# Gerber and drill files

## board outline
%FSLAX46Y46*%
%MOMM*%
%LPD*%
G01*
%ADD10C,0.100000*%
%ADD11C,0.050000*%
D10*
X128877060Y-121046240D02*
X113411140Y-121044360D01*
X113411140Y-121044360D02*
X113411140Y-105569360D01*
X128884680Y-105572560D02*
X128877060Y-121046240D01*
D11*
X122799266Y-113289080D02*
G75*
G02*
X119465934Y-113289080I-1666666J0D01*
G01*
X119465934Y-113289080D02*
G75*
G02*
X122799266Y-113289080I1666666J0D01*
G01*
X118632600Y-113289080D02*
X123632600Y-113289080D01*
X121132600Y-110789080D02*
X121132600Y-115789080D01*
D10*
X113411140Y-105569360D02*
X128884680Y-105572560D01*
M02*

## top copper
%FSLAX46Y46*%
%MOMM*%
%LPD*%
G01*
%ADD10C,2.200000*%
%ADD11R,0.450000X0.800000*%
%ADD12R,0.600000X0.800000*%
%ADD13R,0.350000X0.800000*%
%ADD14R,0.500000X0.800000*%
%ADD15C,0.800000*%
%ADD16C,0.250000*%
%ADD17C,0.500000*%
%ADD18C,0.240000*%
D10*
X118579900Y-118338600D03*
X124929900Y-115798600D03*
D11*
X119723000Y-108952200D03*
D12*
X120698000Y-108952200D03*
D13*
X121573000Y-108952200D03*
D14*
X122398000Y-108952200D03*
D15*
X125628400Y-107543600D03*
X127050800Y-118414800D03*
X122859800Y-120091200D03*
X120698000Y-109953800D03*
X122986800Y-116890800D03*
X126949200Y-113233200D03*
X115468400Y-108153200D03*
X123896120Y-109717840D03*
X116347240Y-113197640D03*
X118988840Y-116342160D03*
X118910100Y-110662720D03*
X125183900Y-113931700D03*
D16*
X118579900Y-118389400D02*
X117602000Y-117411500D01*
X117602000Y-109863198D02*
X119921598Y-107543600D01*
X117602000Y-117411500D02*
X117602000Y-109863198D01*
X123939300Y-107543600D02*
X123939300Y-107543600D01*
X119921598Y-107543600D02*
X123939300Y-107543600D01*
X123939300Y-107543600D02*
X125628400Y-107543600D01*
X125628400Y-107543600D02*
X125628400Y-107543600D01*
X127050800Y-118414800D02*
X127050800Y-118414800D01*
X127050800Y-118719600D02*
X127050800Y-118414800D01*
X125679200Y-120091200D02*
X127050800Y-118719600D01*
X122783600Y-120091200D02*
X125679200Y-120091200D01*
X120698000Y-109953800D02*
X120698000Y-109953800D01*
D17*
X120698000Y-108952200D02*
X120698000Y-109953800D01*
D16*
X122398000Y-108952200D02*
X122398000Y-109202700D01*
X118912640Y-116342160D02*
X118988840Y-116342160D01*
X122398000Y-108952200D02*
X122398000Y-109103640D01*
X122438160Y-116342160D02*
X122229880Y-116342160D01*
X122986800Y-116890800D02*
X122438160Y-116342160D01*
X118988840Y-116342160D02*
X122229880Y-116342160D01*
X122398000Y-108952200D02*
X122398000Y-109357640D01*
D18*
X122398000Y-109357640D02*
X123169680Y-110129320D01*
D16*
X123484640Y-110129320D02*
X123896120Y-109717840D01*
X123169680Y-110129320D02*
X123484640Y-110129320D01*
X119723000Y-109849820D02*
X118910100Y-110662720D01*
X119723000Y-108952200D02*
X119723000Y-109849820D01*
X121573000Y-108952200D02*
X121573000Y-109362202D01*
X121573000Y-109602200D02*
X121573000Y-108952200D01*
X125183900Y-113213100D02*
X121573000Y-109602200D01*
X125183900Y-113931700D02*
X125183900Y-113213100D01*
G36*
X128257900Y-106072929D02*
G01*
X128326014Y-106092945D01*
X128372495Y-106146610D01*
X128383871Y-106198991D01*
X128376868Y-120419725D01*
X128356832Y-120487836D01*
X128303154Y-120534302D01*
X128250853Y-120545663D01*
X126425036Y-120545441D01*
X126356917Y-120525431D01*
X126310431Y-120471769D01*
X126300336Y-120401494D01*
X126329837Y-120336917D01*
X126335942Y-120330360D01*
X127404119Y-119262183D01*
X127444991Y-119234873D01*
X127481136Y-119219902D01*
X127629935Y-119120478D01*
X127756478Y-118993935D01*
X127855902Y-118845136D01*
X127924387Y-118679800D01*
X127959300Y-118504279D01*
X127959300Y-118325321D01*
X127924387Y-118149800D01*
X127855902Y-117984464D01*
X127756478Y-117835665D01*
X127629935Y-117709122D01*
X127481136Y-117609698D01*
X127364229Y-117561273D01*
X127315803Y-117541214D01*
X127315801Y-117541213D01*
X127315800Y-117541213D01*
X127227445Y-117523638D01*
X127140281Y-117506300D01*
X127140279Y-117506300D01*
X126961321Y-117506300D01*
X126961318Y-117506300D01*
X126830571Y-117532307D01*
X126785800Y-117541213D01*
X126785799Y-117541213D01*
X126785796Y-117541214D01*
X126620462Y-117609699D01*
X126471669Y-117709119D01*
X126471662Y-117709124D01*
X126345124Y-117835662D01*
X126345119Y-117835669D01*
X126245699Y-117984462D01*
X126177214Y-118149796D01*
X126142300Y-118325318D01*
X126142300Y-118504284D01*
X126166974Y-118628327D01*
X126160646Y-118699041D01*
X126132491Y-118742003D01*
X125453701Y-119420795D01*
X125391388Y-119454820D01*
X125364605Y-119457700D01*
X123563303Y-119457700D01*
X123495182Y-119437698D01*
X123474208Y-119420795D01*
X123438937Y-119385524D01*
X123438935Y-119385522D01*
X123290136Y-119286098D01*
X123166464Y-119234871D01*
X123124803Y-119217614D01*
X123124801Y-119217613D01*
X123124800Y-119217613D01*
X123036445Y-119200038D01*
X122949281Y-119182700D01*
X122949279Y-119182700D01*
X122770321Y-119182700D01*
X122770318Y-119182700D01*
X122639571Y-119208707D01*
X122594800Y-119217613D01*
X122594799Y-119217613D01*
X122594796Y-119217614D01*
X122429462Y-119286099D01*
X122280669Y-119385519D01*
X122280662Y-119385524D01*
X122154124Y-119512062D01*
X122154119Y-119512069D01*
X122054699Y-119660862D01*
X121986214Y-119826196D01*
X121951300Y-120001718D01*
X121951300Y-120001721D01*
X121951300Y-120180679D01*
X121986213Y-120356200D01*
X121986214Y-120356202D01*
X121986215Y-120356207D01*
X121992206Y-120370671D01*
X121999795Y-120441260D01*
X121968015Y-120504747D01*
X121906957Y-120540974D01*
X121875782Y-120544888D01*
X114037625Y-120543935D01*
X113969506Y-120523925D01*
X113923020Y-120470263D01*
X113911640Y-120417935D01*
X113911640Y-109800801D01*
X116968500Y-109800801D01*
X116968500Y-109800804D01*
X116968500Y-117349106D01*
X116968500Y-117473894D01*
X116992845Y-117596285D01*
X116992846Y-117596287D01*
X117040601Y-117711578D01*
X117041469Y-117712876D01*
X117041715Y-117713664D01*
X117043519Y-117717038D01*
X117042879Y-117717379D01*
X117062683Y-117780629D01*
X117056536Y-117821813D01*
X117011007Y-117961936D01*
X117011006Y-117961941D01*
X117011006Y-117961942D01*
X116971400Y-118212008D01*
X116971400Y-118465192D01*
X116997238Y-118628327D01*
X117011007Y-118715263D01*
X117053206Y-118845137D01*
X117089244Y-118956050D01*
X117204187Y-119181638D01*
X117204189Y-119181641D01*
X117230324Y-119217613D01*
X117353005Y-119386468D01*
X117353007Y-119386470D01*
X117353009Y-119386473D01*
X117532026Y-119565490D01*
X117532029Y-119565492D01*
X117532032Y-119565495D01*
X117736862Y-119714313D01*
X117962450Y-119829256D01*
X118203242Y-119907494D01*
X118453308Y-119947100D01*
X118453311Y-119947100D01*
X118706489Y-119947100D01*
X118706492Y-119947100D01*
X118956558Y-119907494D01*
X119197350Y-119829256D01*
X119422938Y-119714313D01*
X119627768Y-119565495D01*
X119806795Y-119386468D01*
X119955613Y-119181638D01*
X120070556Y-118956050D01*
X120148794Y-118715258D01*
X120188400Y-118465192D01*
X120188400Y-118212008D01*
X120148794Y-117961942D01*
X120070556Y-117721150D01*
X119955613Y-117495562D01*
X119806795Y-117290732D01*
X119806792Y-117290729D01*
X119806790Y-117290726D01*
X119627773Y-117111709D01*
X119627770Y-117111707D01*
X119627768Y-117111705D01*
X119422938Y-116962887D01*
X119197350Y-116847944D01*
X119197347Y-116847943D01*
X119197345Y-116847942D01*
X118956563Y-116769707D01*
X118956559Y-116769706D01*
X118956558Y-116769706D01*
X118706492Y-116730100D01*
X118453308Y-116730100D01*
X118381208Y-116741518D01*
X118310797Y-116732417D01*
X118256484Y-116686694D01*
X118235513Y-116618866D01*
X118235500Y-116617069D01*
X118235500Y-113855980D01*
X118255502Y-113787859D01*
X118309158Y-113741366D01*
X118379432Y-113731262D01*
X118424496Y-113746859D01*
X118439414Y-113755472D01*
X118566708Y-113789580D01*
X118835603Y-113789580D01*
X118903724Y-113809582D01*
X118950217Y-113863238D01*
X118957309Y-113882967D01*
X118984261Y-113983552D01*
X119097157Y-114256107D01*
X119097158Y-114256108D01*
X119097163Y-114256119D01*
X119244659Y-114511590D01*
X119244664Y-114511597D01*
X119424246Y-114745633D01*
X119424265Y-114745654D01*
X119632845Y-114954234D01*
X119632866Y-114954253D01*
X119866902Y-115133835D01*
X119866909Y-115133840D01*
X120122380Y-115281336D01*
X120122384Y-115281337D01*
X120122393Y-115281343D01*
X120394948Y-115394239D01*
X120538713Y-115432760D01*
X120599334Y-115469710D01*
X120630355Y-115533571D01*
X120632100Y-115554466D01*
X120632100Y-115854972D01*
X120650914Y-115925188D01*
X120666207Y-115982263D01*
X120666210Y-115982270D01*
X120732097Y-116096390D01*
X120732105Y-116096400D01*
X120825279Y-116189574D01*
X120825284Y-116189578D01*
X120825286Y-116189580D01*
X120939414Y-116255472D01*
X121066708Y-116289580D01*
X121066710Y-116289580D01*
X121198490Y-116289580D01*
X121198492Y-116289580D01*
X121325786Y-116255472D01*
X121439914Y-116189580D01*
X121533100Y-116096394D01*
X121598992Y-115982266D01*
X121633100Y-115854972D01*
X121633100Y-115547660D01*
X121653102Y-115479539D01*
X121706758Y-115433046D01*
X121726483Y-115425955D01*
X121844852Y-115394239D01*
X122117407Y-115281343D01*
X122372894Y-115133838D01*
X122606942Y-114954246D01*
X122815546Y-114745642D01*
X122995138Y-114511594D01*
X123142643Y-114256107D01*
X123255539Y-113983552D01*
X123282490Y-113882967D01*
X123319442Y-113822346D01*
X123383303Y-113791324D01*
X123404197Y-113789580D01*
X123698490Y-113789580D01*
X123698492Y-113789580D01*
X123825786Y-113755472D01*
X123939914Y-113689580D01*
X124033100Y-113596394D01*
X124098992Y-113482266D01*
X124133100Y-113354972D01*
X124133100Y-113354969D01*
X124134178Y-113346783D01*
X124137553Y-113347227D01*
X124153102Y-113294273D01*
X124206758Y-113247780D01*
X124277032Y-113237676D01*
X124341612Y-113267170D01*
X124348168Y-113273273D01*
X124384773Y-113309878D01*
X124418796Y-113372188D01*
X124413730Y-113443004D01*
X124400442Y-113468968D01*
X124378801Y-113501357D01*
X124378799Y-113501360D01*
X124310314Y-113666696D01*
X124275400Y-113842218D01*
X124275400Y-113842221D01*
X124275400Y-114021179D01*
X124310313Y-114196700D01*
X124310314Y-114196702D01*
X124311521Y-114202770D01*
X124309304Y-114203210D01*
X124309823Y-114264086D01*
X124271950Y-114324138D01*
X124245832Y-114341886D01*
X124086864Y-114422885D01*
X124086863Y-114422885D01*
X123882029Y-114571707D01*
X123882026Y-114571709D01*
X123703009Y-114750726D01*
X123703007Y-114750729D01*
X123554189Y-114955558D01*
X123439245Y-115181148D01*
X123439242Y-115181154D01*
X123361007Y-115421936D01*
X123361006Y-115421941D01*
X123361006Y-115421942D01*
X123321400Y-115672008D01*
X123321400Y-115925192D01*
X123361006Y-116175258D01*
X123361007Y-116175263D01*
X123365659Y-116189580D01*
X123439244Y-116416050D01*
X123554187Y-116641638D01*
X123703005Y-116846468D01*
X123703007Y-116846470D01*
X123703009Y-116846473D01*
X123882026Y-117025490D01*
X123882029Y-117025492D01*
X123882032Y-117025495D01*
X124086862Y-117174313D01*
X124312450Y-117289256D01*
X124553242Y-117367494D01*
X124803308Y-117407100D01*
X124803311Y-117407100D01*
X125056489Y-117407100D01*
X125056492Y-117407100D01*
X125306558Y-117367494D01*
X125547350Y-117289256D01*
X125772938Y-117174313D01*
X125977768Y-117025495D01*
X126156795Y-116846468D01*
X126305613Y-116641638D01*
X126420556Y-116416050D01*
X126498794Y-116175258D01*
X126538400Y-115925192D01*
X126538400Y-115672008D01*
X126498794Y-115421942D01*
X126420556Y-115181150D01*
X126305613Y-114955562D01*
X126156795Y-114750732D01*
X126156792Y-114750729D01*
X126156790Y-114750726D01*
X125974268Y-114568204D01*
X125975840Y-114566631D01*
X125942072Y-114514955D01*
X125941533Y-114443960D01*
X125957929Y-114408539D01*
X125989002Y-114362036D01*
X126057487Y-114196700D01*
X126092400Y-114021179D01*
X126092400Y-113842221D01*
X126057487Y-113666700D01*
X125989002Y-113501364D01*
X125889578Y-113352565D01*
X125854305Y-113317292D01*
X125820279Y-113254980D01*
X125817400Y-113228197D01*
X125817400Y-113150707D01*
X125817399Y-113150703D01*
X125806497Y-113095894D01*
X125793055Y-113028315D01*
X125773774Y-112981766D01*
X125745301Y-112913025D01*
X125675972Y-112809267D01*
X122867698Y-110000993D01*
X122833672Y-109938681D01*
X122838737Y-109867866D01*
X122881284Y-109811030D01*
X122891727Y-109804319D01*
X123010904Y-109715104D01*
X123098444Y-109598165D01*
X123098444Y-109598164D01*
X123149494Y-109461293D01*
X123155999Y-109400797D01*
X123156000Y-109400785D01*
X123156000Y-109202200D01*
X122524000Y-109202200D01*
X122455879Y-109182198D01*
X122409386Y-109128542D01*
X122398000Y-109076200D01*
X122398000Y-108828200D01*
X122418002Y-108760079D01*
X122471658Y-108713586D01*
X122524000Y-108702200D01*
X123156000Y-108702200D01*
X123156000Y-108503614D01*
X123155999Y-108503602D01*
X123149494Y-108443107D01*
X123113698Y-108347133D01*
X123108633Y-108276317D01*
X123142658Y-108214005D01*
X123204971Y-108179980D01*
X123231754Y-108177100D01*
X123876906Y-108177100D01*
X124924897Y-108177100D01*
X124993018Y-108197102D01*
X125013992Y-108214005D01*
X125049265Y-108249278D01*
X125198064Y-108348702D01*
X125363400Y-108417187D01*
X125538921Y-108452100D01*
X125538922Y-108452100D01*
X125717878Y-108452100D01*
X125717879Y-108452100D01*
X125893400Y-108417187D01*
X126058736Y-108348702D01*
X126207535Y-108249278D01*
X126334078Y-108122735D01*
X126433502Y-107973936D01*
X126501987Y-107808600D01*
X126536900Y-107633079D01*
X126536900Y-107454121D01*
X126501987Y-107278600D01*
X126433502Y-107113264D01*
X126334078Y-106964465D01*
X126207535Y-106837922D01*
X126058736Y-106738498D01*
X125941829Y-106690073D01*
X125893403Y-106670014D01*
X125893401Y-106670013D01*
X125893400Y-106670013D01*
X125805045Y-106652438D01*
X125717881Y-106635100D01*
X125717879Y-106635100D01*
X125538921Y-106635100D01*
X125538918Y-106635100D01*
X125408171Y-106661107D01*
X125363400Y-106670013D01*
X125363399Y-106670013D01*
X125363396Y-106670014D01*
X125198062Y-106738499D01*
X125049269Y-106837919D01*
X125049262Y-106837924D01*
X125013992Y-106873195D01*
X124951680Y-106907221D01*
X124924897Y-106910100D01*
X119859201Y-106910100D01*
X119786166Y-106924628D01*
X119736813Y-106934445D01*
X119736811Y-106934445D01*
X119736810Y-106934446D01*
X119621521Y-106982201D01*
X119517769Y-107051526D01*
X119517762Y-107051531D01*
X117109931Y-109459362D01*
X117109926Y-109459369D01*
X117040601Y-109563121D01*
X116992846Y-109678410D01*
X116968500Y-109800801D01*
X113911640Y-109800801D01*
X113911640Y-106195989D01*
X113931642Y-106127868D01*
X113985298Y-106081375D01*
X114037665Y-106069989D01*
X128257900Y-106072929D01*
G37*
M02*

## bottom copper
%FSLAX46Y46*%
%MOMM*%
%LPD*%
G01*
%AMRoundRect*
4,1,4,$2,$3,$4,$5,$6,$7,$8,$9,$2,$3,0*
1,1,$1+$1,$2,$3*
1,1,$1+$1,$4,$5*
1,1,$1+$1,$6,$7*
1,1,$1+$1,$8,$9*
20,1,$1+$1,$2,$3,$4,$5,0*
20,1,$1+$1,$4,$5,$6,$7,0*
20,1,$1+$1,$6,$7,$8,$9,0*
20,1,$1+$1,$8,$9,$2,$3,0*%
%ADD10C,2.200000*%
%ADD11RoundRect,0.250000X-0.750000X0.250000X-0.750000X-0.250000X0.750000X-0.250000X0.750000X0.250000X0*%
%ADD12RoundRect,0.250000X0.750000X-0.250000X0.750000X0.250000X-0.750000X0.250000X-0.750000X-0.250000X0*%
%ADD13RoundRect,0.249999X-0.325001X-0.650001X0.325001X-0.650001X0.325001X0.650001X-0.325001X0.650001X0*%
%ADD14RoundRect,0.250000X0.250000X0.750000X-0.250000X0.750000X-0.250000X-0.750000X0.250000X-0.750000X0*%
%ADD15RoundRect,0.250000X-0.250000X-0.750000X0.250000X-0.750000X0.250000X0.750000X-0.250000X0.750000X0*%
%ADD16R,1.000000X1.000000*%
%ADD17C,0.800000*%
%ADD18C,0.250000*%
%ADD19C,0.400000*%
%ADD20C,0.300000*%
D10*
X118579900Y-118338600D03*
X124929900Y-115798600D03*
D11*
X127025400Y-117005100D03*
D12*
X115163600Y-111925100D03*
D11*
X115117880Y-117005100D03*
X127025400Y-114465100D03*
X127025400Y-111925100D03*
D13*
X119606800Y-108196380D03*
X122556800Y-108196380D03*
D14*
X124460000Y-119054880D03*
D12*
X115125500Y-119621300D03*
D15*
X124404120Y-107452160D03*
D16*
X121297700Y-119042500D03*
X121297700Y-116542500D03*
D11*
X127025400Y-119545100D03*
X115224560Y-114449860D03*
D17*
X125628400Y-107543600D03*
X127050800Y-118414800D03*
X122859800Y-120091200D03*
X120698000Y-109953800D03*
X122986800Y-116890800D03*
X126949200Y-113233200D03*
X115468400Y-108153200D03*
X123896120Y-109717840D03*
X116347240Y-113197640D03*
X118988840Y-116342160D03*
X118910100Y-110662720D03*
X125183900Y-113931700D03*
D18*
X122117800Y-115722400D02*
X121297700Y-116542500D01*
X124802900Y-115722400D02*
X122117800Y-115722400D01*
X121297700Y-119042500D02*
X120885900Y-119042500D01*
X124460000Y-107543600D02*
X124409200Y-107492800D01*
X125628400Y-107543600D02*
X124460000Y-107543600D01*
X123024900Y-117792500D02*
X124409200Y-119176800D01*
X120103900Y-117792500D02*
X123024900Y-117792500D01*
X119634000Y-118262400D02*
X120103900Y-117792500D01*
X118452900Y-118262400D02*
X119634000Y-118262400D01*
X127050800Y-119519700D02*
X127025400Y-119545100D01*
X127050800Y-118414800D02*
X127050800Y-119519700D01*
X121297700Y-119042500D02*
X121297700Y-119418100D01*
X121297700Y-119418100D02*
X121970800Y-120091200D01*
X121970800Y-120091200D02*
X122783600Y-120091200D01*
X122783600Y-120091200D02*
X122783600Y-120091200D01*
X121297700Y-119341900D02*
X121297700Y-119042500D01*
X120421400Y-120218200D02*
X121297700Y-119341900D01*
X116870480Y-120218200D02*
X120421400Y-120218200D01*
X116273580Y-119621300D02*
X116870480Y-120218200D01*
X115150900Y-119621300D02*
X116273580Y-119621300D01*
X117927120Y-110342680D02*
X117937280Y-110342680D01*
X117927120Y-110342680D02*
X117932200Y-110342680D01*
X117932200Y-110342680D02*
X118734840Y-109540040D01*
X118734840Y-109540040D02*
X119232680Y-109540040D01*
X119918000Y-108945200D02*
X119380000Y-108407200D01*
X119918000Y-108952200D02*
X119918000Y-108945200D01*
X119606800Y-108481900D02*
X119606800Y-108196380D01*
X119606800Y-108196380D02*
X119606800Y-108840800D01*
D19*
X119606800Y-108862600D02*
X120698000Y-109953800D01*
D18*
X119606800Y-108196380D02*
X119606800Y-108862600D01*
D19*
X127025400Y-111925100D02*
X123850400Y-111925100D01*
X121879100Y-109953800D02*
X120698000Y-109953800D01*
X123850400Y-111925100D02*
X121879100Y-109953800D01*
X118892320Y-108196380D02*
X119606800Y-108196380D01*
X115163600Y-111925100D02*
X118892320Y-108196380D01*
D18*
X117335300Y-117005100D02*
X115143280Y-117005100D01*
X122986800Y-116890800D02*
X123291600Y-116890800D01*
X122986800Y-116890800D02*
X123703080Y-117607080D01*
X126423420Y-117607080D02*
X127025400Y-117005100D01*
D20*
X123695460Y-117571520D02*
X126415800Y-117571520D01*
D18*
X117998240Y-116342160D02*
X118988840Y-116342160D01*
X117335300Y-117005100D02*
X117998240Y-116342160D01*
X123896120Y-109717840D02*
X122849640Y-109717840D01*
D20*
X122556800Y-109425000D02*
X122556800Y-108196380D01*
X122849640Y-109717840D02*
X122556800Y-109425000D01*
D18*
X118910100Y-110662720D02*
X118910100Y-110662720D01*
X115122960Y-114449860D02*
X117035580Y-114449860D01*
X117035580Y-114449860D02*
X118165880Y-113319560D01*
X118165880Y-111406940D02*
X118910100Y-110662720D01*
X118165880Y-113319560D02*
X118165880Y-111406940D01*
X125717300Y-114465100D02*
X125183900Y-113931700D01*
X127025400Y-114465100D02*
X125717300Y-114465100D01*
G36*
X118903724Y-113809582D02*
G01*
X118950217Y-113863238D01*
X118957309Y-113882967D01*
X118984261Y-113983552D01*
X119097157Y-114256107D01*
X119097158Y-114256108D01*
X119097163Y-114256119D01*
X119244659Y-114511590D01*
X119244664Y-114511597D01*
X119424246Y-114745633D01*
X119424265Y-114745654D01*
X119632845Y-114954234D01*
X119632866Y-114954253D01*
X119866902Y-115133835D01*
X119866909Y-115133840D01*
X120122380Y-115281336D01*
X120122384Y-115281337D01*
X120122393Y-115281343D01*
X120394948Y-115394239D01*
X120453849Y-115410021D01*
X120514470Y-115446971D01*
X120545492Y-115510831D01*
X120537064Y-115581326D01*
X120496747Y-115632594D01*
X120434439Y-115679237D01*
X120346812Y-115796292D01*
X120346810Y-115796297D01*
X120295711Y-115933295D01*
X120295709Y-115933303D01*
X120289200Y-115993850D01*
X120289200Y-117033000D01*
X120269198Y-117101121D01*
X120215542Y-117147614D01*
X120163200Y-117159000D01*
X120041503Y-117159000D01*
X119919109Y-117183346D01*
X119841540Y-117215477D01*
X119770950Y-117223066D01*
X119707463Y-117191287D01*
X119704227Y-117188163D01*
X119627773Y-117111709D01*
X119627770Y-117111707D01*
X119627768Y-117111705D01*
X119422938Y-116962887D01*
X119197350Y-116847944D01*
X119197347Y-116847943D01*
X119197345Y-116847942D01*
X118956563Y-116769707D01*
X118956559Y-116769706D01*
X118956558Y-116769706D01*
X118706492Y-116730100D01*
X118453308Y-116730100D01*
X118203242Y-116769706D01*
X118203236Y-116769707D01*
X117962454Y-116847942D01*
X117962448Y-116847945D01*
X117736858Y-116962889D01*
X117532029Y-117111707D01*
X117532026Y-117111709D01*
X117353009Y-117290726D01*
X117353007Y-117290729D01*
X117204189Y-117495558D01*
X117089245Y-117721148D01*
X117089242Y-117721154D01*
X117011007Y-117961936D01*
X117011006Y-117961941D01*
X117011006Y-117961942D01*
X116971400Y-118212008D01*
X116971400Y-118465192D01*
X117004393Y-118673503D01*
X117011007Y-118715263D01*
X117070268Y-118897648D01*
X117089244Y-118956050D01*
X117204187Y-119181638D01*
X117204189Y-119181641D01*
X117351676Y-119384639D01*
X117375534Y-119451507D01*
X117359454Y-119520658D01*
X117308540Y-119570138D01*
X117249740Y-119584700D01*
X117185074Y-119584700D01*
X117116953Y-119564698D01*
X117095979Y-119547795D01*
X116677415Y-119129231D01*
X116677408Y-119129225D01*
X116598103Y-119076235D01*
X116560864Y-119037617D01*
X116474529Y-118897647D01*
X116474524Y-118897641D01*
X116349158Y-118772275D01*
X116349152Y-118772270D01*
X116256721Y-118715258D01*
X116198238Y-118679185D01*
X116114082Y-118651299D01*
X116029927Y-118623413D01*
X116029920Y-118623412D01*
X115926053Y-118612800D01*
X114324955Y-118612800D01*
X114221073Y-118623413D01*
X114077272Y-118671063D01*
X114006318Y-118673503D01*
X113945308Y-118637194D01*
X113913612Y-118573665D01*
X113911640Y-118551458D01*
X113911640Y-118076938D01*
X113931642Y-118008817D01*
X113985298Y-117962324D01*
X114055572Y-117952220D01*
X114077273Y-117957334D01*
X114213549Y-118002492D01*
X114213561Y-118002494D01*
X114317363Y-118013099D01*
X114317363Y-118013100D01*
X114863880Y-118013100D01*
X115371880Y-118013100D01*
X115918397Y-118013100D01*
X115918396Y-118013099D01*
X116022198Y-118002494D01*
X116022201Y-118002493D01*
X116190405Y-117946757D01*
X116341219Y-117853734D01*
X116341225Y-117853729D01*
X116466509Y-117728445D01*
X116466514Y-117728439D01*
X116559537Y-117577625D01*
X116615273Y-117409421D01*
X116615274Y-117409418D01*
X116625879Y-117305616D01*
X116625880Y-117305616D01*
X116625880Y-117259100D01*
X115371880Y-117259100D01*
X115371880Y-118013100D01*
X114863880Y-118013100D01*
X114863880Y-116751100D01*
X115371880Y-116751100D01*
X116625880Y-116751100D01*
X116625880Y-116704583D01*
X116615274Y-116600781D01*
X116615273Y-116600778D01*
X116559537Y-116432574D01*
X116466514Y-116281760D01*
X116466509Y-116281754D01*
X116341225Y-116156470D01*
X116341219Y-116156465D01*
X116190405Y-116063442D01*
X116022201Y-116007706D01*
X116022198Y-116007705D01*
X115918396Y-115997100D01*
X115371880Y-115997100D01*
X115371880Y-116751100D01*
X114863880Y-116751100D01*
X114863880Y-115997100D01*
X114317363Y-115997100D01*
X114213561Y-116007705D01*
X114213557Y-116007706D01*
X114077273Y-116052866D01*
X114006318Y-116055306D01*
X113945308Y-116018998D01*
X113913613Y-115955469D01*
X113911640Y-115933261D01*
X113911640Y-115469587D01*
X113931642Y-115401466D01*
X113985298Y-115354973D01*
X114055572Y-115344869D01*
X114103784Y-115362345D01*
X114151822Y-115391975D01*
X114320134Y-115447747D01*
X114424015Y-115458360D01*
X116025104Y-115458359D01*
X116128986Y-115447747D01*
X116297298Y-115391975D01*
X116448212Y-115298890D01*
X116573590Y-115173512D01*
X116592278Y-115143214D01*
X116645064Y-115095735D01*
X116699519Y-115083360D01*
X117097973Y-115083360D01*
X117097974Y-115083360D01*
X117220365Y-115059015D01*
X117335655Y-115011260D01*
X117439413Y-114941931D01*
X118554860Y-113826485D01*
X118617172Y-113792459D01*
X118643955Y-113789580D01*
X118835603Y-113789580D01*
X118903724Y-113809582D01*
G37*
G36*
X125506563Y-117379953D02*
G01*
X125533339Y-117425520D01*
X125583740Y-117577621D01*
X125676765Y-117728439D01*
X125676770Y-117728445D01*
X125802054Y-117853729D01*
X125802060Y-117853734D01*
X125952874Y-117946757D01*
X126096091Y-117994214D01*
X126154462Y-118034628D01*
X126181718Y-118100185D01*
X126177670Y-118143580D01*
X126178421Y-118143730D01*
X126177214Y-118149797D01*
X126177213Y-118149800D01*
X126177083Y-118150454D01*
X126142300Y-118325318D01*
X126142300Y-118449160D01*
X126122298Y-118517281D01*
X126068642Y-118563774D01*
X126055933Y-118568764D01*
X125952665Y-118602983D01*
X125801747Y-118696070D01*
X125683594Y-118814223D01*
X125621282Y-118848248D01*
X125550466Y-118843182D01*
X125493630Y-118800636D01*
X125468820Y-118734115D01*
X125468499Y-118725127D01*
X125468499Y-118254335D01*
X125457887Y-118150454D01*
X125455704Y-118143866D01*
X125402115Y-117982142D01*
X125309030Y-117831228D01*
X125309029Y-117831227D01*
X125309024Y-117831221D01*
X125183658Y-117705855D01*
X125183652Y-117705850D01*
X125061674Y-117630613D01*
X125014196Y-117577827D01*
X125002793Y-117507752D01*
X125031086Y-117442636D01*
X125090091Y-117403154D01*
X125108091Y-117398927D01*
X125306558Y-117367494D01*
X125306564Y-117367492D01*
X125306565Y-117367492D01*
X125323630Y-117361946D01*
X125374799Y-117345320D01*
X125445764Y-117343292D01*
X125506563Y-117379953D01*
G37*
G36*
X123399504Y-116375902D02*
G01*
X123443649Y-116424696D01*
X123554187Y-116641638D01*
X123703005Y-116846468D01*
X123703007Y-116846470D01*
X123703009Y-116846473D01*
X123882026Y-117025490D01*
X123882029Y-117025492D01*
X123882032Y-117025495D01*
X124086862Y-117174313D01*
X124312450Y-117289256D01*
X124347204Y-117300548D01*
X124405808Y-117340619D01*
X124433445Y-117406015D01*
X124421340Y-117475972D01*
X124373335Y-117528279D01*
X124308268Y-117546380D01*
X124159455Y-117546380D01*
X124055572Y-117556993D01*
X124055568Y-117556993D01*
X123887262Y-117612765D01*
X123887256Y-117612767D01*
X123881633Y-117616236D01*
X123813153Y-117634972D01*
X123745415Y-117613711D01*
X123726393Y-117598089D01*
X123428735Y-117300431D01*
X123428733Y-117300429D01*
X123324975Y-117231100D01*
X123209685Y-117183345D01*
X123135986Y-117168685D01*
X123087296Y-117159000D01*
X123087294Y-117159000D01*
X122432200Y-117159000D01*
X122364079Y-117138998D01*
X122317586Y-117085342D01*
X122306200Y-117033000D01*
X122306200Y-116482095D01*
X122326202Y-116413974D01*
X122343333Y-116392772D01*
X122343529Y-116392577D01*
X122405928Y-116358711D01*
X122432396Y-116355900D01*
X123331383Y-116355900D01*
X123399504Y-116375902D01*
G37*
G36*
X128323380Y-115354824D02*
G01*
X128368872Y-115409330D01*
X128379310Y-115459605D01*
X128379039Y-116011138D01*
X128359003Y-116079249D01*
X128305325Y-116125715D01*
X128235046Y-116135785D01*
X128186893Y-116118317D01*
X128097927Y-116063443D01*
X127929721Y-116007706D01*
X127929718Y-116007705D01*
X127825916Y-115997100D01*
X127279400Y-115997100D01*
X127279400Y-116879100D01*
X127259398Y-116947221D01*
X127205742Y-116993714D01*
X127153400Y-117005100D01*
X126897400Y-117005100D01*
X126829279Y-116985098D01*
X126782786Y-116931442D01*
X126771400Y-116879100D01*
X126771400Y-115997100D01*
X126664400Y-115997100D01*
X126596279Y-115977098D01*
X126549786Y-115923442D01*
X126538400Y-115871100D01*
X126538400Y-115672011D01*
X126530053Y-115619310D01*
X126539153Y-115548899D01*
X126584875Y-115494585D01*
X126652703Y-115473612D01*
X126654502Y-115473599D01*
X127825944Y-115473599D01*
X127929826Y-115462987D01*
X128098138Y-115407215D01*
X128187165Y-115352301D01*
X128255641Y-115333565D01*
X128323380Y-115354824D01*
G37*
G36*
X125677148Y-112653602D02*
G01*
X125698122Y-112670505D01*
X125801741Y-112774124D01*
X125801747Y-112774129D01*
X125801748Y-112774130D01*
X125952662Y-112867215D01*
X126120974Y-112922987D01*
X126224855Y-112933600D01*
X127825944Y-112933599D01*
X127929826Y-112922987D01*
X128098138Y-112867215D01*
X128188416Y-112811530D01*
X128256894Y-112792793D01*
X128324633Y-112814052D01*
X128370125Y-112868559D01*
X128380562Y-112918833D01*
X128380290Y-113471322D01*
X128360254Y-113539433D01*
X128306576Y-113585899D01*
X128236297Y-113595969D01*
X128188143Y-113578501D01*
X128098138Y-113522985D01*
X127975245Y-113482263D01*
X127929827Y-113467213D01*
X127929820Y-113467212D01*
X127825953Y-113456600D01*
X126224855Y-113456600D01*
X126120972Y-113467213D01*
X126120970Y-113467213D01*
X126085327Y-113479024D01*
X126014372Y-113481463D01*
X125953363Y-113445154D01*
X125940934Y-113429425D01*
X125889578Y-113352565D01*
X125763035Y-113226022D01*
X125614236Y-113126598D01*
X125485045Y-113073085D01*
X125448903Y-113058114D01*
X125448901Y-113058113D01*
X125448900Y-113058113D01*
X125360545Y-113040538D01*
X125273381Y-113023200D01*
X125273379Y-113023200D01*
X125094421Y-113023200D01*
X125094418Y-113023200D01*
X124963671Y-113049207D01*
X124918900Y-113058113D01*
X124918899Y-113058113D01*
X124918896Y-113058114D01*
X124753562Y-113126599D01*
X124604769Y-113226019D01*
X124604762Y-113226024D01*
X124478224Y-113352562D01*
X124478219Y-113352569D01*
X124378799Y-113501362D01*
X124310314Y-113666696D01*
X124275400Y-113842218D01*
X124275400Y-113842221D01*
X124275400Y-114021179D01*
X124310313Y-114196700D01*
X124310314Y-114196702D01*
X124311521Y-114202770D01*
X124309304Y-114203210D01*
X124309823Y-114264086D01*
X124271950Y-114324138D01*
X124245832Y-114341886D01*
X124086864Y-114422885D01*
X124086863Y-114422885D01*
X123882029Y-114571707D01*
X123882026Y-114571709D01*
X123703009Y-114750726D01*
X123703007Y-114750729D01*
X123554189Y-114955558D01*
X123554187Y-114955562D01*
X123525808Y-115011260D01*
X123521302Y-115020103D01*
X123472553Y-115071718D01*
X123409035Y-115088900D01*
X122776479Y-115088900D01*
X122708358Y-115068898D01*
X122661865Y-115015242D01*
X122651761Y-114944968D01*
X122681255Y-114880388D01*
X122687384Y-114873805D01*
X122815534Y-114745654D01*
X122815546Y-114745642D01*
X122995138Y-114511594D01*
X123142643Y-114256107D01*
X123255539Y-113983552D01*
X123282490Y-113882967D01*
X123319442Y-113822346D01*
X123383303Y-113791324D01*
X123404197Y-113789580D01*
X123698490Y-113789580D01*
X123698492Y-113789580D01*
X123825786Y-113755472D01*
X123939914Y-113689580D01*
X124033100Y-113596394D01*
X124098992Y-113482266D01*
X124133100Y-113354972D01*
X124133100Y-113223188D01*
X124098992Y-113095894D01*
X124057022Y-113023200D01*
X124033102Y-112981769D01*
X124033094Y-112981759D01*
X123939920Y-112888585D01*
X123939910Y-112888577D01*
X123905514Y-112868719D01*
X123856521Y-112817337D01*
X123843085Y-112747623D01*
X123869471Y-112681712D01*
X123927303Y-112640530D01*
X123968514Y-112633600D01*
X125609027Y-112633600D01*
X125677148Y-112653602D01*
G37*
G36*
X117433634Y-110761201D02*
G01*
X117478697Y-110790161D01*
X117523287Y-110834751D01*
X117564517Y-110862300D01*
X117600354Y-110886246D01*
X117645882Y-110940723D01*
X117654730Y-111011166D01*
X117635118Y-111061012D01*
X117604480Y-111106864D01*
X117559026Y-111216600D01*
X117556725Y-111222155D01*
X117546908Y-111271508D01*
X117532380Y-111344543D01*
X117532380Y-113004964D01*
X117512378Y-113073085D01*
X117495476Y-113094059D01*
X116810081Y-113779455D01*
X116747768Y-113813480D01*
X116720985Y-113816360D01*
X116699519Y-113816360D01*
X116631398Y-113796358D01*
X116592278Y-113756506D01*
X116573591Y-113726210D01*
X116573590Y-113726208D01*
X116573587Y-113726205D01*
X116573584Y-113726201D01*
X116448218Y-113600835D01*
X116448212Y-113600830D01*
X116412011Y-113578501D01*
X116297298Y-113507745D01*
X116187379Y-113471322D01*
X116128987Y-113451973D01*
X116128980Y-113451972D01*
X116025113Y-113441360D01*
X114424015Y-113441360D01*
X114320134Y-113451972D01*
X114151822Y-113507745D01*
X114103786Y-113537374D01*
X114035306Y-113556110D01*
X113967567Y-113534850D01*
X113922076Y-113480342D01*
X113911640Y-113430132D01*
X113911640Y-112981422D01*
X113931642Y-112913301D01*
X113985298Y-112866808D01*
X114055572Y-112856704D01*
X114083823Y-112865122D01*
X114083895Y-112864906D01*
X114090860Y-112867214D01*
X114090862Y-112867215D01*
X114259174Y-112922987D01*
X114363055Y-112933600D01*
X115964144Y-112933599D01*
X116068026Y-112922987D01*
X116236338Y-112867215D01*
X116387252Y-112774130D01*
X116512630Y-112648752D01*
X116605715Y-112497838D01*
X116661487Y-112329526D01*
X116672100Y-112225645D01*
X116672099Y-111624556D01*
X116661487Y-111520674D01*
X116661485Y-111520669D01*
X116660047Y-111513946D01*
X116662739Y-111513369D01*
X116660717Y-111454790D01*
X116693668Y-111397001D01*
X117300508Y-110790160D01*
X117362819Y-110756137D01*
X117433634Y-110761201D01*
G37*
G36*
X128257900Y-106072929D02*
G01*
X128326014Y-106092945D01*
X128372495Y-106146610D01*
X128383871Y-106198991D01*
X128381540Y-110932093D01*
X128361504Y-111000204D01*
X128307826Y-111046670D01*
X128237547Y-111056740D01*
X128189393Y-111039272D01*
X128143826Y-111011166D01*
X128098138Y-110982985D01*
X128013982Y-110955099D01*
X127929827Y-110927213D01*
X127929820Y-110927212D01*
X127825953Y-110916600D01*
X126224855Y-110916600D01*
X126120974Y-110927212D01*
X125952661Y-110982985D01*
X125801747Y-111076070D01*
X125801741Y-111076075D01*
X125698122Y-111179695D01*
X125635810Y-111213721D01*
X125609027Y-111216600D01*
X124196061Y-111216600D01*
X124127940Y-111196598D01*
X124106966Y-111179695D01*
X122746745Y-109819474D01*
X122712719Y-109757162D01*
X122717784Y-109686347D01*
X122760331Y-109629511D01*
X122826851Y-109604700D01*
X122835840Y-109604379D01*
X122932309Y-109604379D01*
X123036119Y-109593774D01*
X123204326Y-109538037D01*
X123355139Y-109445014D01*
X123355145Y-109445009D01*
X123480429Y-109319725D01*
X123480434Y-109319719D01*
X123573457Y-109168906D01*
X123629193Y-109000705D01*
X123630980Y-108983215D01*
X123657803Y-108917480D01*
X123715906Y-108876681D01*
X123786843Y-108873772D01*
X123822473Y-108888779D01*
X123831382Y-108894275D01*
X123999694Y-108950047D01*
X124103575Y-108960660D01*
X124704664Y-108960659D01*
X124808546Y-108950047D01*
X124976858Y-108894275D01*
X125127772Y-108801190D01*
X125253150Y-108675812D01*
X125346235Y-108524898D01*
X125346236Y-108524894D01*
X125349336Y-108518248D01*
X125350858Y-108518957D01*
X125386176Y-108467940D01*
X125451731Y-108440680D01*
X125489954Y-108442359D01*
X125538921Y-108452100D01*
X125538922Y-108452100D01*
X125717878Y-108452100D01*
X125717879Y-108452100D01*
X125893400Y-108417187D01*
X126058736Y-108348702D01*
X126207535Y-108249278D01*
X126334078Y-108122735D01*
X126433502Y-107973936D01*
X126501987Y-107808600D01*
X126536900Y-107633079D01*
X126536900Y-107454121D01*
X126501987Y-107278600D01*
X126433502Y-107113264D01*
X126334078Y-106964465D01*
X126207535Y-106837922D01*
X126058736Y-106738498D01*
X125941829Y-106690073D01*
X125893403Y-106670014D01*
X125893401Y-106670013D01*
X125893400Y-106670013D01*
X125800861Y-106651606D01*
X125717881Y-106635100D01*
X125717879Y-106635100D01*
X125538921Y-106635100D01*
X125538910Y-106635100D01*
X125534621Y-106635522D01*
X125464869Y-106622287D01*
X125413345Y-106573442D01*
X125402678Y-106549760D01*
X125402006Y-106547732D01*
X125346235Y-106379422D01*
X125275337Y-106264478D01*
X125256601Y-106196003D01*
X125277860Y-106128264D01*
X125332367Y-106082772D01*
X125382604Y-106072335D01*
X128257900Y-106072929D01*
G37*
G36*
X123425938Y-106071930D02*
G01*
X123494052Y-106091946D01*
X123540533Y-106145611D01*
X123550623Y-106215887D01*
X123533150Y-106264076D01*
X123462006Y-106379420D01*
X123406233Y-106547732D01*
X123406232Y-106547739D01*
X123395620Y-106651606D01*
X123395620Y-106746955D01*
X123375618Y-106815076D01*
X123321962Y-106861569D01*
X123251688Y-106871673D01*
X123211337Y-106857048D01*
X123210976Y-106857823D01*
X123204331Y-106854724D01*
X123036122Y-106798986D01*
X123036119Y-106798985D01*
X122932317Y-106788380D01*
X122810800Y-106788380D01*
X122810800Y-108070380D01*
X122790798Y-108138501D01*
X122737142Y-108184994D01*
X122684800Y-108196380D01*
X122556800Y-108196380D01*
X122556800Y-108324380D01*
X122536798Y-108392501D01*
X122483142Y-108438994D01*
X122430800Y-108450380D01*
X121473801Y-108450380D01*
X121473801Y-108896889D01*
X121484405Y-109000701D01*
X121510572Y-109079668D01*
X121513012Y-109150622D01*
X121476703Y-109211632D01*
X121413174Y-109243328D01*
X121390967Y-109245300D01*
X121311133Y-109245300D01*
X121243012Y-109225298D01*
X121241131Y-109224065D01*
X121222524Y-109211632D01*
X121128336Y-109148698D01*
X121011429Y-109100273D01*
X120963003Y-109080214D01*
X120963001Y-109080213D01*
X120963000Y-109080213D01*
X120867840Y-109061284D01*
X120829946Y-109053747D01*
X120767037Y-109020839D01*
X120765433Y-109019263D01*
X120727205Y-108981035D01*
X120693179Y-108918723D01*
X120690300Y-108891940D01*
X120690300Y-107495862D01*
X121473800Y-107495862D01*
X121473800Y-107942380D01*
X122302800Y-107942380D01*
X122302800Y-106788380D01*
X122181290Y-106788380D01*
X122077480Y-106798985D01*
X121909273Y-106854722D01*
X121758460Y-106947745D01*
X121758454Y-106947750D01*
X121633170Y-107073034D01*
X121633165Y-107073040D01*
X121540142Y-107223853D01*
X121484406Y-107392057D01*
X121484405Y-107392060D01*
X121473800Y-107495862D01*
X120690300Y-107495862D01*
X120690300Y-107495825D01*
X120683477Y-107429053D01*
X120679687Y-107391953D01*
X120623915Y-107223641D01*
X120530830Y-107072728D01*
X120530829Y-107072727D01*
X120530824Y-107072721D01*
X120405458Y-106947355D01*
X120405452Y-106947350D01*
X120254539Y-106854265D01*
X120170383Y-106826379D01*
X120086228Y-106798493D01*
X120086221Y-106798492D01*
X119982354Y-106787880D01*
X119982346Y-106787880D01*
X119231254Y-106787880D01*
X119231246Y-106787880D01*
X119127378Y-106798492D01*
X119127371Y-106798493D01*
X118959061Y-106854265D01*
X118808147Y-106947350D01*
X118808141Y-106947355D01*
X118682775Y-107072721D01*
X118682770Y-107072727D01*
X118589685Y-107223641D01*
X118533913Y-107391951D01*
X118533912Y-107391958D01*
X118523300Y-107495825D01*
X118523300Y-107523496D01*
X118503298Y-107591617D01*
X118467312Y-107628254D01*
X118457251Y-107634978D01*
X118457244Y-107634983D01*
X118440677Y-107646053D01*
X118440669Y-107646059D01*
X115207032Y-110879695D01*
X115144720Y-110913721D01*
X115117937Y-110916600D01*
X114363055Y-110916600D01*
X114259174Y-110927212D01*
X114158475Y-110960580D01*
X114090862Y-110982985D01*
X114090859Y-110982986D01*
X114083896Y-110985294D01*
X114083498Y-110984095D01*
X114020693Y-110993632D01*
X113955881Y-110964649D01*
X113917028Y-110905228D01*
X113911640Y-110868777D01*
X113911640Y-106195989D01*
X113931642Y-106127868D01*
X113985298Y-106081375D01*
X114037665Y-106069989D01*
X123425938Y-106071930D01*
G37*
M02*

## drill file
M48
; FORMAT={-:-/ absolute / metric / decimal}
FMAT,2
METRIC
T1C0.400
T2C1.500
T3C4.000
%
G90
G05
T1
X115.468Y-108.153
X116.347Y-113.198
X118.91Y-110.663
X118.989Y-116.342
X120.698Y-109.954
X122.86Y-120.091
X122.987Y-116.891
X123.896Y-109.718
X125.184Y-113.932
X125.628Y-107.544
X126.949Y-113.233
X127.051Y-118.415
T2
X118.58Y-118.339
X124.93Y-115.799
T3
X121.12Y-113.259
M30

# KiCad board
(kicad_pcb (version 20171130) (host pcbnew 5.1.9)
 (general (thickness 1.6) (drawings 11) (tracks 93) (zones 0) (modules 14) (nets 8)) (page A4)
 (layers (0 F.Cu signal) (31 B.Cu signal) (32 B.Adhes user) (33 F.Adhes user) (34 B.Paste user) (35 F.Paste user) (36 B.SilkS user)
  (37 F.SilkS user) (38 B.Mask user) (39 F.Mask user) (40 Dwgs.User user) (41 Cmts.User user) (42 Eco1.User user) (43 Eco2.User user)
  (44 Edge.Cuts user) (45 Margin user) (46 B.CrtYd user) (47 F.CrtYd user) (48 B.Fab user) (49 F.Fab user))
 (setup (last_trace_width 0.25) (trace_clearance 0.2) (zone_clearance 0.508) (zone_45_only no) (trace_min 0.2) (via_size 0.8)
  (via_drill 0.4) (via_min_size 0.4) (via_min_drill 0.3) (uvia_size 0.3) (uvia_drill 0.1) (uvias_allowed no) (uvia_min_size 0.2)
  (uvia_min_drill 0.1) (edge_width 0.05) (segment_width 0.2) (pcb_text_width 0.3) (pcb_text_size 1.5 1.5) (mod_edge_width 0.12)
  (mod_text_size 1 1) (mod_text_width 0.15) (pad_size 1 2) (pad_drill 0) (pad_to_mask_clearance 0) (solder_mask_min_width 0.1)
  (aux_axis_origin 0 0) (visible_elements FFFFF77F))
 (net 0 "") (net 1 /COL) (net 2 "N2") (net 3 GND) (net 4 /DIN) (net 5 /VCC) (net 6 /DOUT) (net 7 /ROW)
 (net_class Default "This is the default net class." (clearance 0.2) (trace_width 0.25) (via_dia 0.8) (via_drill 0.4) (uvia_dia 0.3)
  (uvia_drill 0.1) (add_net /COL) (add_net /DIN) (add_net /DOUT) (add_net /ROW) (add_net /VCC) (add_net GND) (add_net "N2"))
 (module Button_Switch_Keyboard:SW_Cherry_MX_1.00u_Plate (layer F.Cu) (at 118.5799 118.3386 180)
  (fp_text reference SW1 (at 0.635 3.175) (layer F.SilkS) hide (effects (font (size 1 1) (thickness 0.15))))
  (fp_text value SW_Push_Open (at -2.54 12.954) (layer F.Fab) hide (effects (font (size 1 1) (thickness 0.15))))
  (pad 1 thru_hole circle (at 0 0 180) (size 2.2 2.2) (drill 1.5) (layers *.Cu *.Mask) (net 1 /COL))
  (pad 2 thru_hole circle (at -6.35 2.54 180) (size 2.2 2.2) (drill 1.5) (layers *.Cu *.Mask) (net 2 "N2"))
  (pad "" np_thru_hole circle (at -2.54 5.08 180) (size 4 4) (drill 4) (layers *.Cu *.Mask)))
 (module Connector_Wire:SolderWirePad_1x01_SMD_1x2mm (layer B.Cu) (at 127.0254 117.0051 270)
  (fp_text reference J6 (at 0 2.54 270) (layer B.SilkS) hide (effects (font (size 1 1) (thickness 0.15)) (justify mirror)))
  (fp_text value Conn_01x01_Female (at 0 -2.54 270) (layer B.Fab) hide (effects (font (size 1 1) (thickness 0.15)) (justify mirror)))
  (pad 1 smd roundrect (at 0 0 270) (size 1 2) (layers B.Cu B.Paste B.Mask) (roundrect_rratio 0.25) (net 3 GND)))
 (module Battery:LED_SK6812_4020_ (layer F.Cu) (at 121.158 107.7722)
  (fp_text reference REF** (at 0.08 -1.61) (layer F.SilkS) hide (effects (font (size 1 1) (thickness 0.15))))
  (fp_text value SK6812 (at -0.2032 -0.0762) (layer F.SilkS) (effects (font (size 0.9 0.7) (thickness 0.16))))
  (pad 1 smd rect (at -1.435 1.18) (size 0.45 0.8) (layers F.Cu F.Paste F.Mask) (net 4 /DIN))
  (pad 2 smd rect (at -0.46 1.18) (size 0.6 0.8) (layers F.Cu F.Paste F.Mask) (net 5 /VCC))
  (pad 3 smd rect (at 0.415 1.18) (size 0.35 0.8) (layers F.Cu F.Paste F.Mask) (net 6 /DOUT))
  (pad 4 smd rect (at 1.24 1.18) (size 0.5 0.8) (layers F.Cu F.Paste F.Mask) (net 3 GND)))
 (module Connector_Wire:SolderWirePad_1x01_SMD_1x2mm (layer B.Cu) (at 115.1636 111.9251 90)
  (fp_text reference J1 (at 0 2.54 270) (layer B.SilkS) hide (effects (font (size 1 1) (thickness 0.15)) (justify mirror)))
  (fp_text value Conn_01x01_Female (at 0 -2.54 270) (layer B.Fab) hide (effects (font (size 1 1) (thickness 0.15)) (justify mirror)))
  (pad 1 smd roundrect (at 0 0 90) (size 1 2) (layers B.Cu B.Paste B.Mask) (roundrect_rratio 0.25) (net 5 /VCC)))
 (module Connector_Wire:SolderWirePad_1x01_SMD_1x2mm (layer B.Cu) (at 115.11788 117.0051 270)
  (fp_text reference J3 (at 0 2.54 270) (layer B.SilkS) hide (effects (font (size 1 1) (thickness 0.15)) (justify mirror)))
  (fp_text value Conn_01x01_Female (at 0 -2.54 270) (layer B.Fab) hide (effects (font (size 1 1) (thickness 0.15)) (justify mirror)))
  (pad 1 smd roundrect (at 0 0 270) (size 1 2) (layers B.Cu B.Paste B.Mask) (roundrect_rratio 0.25) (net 3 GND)))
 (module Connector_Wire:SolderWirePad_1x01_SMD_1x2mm (layer B.Cu) (at 127.0254 114.4651 270)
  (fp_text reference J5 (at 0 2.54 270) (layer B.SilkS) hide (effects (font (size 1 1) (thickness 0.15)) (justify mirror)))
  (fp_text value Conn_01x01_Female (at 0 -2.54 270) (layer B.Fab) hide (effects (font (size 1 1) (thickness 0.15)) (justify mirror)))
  (pad 1 smd roundrect (at 0 0 270) (size 1 2) (layers B.Cu B.Paste B.Mask) (roundrect_rratio 0.25) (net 6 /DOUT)))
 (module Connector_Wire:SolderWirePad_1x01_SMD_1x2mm (layer B.Cu) (at 127.0254 111.9251 270)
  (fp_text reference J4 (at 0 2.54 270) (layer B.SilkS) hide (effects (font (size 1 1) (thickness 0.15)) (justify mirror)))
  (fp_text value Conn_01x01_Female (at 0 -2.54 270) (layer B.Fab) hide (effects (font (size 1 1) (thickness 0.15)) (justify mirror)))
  (pad 1 smd roundrect (at 0 0 270) (size 1 2) (layers B.Cu B.Paste B.Mask) (roundrect_rratio 0.25) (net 5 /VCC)))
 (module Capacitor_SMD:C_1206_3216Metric (layer B.Cu) (at 121.0818 108.19638)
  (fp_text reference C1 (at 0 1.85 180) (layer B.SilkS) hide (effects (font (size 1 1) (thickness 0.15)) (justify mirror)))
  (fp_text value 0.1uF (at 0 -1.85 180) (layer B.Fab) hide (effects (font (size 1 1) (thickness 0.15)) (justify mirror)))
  (pad 1 smd roundrect (at -1.475 0) (size 1.15 1.8) (layers B.Cu B.Paste B.Mask) (roundrect_rratio 0.2173904347826087) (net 5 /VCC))
  (pad 2 smd roundrect (at 1.475 0) (size 1.15 1.8) (layers B.Cu B.Paste B.Mask) (roundrect_rratio 0.2173904347826087) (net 3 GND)))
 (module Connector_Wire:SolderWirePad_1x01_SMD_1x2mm (layer B.Cu) (at 124.46 119.05488 180)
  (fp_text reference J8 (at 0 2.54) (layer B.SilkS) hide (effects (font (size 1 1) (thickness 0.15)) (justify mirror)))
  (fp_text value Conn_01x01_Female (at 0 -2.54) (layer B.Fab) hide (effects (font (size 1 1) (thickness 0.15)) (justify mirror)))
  (pad 1 smd roundrect (at 0 0 180) (size 1 2) (layers B.Cu B.Paste B.Mask) (roundrect_rratio 0.25) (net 1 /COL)))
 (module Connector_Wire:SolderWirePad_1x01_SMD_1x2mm (layer B.Cu) (at 115.1255 119.6213 90)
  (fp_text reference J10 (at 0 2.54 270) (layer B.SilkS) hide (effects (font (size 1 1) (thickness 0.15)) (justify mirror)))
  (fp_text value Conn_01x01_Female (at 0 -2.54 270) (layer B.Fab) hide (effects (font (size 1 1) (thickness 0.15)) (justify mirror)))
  (pad 1 smd roundrect (at 0 0 90) (size 1 2) (layers B.Cu B.Paste B.Mask) (roundrect_rratio 0.25) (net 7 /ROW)))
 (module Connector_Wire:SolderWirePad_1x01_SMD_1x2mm (layer B.Cu) (at 124.40412 107.45216)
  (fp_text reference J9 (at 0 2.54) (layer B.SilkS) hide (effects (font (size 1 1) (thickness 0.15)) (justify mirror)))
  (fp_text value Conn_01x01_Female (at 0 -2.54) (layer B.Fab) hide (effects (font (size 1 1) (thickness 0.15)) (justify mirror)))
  (pad 1 smd roundrect (at 0 0) (size 1 2) (layers B.Cu B.Paste B.Mask) (roundrect_rratio 0.25) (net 1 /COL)))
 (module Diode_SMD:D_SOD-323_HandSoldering (layer B.Cu) (at 121.2977 117.7925 90)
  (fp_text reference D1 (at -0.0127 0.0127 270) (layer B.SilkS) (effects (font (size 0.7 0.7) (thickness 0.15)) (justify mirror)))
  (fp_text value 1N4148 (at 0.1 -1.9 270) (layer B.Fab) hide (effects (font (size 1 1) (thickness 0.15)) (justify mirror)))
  (pad 1 smd rect (at -1.25 0 90) (size 1 1) (layers B.Cu B.Paste B.Mask) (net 7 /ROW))
  (pad 2 smd rect (at 1.25 0 90) (size 1 1) (layers B.Cu B.Paste B.Mask) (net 2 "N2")))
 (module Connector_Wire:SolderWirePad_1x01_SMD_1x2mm (layer B.Cu) (at 127.0254 119.5451 270)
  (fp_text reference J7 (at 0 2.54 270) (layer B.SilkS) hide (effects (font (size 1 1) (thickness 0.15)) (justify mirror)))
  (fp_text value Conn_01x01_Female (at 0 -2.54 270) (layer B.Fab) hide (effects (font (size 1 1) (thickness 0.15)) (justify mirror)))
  (pad 1 smd roundrect (at 0 0 270) (size 1 2) (layers B.Cu B.Paste B.Mask) (roundrect_rratio 0.25) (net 7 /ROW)))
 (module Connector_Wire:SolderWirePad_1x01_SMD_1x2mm (layer B.Cu) (at 115.22456 114.44986 270)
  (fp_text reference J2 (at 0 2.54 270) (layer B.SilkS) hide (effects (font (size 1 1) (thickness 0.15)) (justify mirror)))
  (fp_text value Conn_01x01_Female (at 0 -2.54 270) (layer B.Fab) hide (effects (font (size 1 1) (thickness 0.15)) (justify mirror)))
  (pad 1 smd roundrect (at 0 0 270) (size 1 2) (layers B.Cu B.Paste B.Mask) (roundrect_rratio 0.25) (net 4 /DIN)))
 (gr_line (start 128.87706 121.04624) (end 113.41114 121.04436) (layer Edge.Cuts) (width 0.1))
 (gr_line (start 113.41114 121.04436) (end 113.41114 105.56936) (layer Edge.Cuts) (width 0.1))
 (gr_line (start 128.88468 105.57256) (end 128.87706 121.04624) (layer Edge.Cuts) (width 0.1))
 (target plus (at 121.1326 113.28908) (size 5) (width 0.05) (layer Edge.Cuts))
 (gr_line (start 113.41114 105.56936) (end 128.88468 105.57256) (layer Edge.Cuts) (width 0.1))
 (segment (start 122.1178 115.7224) (end 121.2977 116.5425) (width 0.25) (layer B.Cu) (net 2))
 (segment (start 124.8029 115.7224) (end 122.1178 115.7224) (width 0.25) (layer B.Cu) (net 2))
 (segment (start 121.2977 119.0425) (end 120.8859 119.0425) (width 0.25) (layer B.Cu) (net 7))
 (segment (start 118.5799 118.3894) (end 117.602 117.4115) (width 0.25) (layer F.Cu) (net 1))
 (segment (start 117.602 109.863198) (end 119.921598 107.5436) (width 0.25) (layer F.Cu) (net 1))
 (segment (start 117.602 117.4115) (end 117.602 109.863198) (width 0.25) (layer F.Cu) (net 1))
 (segment (start 123.9393 107.5436) (end 123.9393 107.5436) (width 0.25) (layer F.Cu) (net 1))
 (segment (start 119.921598 107.5436) (end 123.9393 107.5436) (width 0.25) (layer F.Cu) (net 1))
 (segment (start 123.9393 107.5436) (end 125.6284 107.5436) (width 0.25) (layer F.Cu) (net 1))
 (segment (start 125.6284 107.5436) (end 125.6284 107.5436) (width 0.25) (layer F.Cu) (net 1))
 (via (at 125.6284 107.5436) (size 0.8) (drill 0.4) (layers F.Cu B.Cu) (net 1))
 (segment (start 124.46 107.5436) (end 124.4092 107.4928) (width 0.25) (layer B.Cu) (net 1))
 (segment (start 125.6284 107.5436) (end 124.46 107.5436) (width 0.25) (layer B.Cu) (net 1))
 (segment (start 123.0249 117.7925) (end 124.4092 119.1768) (width 0.25) (layer B.Cu) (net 1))
 (segment (start 120.1039 117.7925) (end 123.0249 117.7925) (width 0.25) (layer B.Cu) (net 1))
 (segment (start 119.634 118.2624) (end 120.1039 117.7925) (width 0.25) (layer B.Cu) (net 1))
 (segment (start 118.4529 118.2624) (end 119.634 118.2624) (width 0.25) (layer B.Cu) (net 1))
 (segment (start 127.0508 118.4148) (end 127.0508 118.4148) (width 0.25) (layer F.Cu) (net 7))
 (via (at 127.0508 118.4148) (size 0.8) (drill 0.4) (layers F.Cu B.Cu) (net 7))
 (segment (start 127.0508 119.5197) (end 127.0254 119.5451) (width 0.25) (layer B.Cu) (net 7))
 (segment (start 127.0508 118.4148) (end 127.0508 119.5197) (width 0.25) (layer B.Cu) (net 7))
 (segment (start 121.2977 119.0425) (end 121.2977 119.4181) (width 0.25) (layer B.Cu) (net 7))
 (segment (start 121.2977 119.4181) (end 121.9708 120.0912) (width 0.25) (layer B.Cu) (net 7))
 (segment (start 121.9708 120.0912) (end 122.7836 120.0912) (width 0.25) (layer B.Cu) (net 7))
 (segment (start 122.7836 120.0912) (end 122.7836 120.0912) (width 0.25) (layer B.Cu) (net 7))
 (via (at 122.8598 120.0912) (size 0.8) (drill 0.4) (layers F.Cu B.Cu) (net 7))
 (segment (start 127.0508 118.7196) (end 127.0508 118.4148) (width 0.25) (layer F.Cu) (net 7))
 (segment (start 125.6792 120.0912) (end 127.0508 118.7196) (width 0.25) (layer F.Cu) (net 7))
 (segment (start 122.7836 120.0912) (end 125.6792 120.0912) (width 0.25) (layer F.Cu) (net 7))
 (segment (start 121.2977 119.3419) (end 121.2977 119.0425) (width 0.25) (layer B.Cu) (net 7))
 (segment (start 120.4214 120.2182) (end 121.2977 119.3419) (width 0.25) (layer B.Cu) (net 7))
 (segment (start 116.87048 120.2182) (end 120.4214 120.2182) (width 0.25) (layer B.Cu) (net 7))
 (segment (start 116.27358 119.6213) (end 116.87048 120.2182) (width 0.25) (layer B.Cu) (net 7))
 (segment (start 115.1509 119.6213) (end 116.27358 119.6213) (width 0.25) (layer B.Cu) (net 7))
 (segment (start 117.92712 110.34268) (end 117.93728 110.34268) (width 0.25) (layer B.Cu) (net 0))
 (segment (start 117.92712 110.34268) (end 117.9322 110.34268) (width 0.25) (layer B.Cu) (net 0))
 (segment (start 117.9322 110.34268) (end 118.73484 109.54004) (width 0.25) (layer B.Cu) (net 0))
 (segment (start 118.73484 109.54004) (end 119.23268 109.54004) (width 0.25) (layer B.Cu) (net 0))
 (segment (start 119.918 108.9452) (end 119.38 108.4072) (width 0.25) (layer B.Cu) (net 5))
 (segment (start 119.918 108.9522) (end 119.918 108.9452) (width 0.25) (layer B.Cu) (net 5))
 (segment (start 119.6068 108.4819) (end 119.6068 108.19638) (width 0.25) (layer B.Cu) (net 5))
 (segment (start 120.698 109.9538) (end 120.698 109.9538) (width 0.25) (layer F.Cu) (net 5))
 (via (at 120.698 109.9538) (size 0.8) (drill 0.4) (layers F.Cu B.Cu) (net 5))
 (segment (start 120.698 108.9522) (end 120.698 109.9538) (width 0.5) (layer F.Cu) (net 5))
 (segment (start 119.6068 108.19638) (end 119.6068 108.8408) (width 0.25) (layer B.Cu) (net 5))
 (segment (start 119.6068 108.8626) (end 120.698 109.9538) (width 0.4) (layer B.Cu) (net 5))
 (segment (start 119.6068 108.19638) (end 119.6068 108.8626) (width 0.25) (layer B.Cu) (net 5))
 (segment (start 127.0254 111.9251) (end 123.8504 111.9251) (width 0.4) (layer B.Cu) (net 5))
 (segment (start 121.8791 109.9538) (end 120.698 109.9538) (width 0.4) (layer B.Cu) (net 5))
 (segment (start 123.8504 111.9251) (end 121.8791 109.9538) (width 0.4) (layer B.Cu) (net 5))
 (segment (start 118.89232 108.19638) (end 119.6068 108.19638) (width 0.4) (layer B.Cu) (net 5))
 (segment (start 115.1636 111.9251) (end 118.89232 108.19638) (width 0.4) (layer B.Cu) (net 5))
 (via (at 122.9868 116.8908) (size 0.8) (drill 0.4) (layers F.Cu B.Cu) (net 3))
 (segment (start 122.398 108.9522) (end 122.398 109.2027) (width 0.25) (layer F.Cu) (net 3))
 (segment (start 118.91264 116.34216) (end 118.98884 116.34216) (width 0.25) (layer F.Cu) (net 3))
 (via (at 126.9492 113.2332) (size 0.8) (drill 0.4) (layers F.Cu B.Cu) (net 3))
 (via (at 115.4684 108.1532) (size 0.8) (drill 0.4) (layers F.Cu B.Cu) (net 3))
 (via (at 123.89612 109.71784) (size 0.8) (drill 0.4) (layers F.Cu B.Cu) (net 3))
 (segment (start 117.3353 117.0051) (end 115.14328 117.0051) (width 0.25) (layer B.Cu) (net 3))
 (via (at 116.34724 113.19764) (size 0.8) (drill 0.4) (layers F.Cu B.Cu) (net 3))
 (segment (start 122.9868 116.8908) (end 123.2916 116.8908) (width 0.25) (layer B.Cu) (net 3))
 (segment (start 122.9868 116.8908) (end 123.70308 117.60708) (width 0.25) (layer B.Cu) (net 3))
 (segment (start 126.42342 117.60708) (end 127.0254 117.0051) (width 0.25) (layer B.Cu) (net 3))
 (segment (start 123.69546 117.57152) (end 126.4158 117.57152) (width 0.3) (layer B.Cu) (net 3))
 (segment (start 122.398 108.9522) (end 122.398 109.10364) (width 0.25) (layer F.Cu) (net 3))
 (segment (start 122.43816 116.34216) (end 122.22988 116.34216) (width 0.25) (layer F.Cu) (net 3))
 (segment (start 122.9868 116.8908) (end 122.43816 116.34216) (width 0.25) (layer F.Cu) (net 3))
 (segment (start 118.98884 116.34216) (end 122.22988 116.34216) (width 0.25) (layer F.Cu) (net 3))
 (via (at 118.98884 116.34216) (size 0.8) (drill 0.4) (layers F.Cu B.Cu) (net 3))
 (segment (start 117.99824 116.34216) (end 118.98884 116.34216) (width 0.25) (layer B.Cu) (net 3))
 (segment (start 117.3353 117.0051) (end 117.99824 116.34216) (width 0.25) (layer B.Cu) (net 3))
 (segment (start 123.89612 109.71784) (end 122.84964 109.71784) (width 0.25) (layer B.Cu) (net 3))
 (segment (start 122.5568 109.425) (end 122.5568 108.19638) (width 0.3) (layer B.Cu) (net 3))
 (segment (start 122.84964 109.71784) (end 122.5568 109.425) (width 0.3) (layer B.Cu) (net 3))
 (segment (start 122.398 108.9522) (end 122.398 109.35764) (width 0.25) (layer F.Cu) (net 3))
 (segment (start 122.398 109.35764) (end 123.16968 110.12932) (width 0.24) (layer F.Cu) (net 3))
 (segment (start 123.48464 110.12932) (end 123.89612 109.71784) (width 0.25) (layer F.Cu) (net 3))
 (segment (start 123.16968 110.12932) (end 123.48464 110.12932) (width 0.25) (layer F.Cu) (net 3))
 (segment (start 118.9101 110.66272) (end 118.9101 110.66272) (width 0.25) (layer B.Cu) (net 4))
 (via (at 118.9101 110.66272) (size 0.8) (drill 0.4) (layers F.Cu B.Cu) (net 4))
 (segment (start 119.723 109.84982) (end 118.9101 110.66272) (width 0.25) (layer F.Cu) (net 4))
 (segment (start 119.723 108.9522) (end 119.723 109.84982) (width 0.25) (layer F.Cu) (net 4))
 (segment (start 115.12296 114.44986) (end 117.03558 114.44986) (width 0.25) (layer B.Cu) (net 4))
 (segment (start 117.03558 114.44986) (end 118.16588 113.31956) (width 0.25) (layer B.Cu) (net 4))
 (segment (start 118.16588 111.40694) (end 118.9101 110.66272) (width 0.25) (layer B.Cu) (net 4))
 (segment (start 118.16588 113.31956) (end 118.16588 111.40694) (width 0.25) (layer B.Cu) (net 4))
 (via (at 125.1839 113.9317) (size 0.8) (drill 0.4) (layers F.Cu B.Cu) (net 6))
 (segment (start 121.573 108.9522) (end 121.573 109.362202) (width 0.25) (layer F.Cu) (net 6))
 (segment (start 125.7173 114.4651) (end 125.1839 113.9317) (width 0.25) (layer B.Cu) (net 6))
 (segment (start 127.0254 114.4651) (end 125.7173 114.4651) (width 0.25) (layer B.Cu) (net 6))
 (segment (start 121.573 109.6022) (end 121.573 108.9522) (width 0.25) (layer F.Cu) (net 6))
 (segment (start 125.1839 113.2131) (end 121.573 109.6022) (width 0.25) (layer F.Cu) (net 6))
 (segment (start 125.1839 113.9317) (end 125.1839 113.2131) (width 0.25) (layer F.Cu) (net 6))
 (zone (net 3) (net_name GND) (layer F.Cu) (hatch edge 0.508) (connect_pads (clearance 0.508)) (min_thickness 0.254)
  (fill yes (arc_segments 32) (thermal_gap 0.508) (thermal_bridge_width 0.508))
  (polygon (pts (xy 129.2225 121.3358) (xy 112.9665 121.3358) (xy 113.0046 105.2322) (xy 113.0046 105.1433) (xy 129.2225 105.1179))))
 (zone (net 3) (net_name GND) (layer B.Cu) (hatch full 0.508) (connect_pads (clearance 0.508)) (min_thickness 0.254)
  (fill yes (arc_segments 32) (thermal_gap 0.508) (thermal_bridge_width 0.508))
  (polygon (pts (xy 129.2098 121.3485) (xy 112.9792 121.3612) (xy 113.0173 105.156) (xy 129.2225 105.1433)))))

